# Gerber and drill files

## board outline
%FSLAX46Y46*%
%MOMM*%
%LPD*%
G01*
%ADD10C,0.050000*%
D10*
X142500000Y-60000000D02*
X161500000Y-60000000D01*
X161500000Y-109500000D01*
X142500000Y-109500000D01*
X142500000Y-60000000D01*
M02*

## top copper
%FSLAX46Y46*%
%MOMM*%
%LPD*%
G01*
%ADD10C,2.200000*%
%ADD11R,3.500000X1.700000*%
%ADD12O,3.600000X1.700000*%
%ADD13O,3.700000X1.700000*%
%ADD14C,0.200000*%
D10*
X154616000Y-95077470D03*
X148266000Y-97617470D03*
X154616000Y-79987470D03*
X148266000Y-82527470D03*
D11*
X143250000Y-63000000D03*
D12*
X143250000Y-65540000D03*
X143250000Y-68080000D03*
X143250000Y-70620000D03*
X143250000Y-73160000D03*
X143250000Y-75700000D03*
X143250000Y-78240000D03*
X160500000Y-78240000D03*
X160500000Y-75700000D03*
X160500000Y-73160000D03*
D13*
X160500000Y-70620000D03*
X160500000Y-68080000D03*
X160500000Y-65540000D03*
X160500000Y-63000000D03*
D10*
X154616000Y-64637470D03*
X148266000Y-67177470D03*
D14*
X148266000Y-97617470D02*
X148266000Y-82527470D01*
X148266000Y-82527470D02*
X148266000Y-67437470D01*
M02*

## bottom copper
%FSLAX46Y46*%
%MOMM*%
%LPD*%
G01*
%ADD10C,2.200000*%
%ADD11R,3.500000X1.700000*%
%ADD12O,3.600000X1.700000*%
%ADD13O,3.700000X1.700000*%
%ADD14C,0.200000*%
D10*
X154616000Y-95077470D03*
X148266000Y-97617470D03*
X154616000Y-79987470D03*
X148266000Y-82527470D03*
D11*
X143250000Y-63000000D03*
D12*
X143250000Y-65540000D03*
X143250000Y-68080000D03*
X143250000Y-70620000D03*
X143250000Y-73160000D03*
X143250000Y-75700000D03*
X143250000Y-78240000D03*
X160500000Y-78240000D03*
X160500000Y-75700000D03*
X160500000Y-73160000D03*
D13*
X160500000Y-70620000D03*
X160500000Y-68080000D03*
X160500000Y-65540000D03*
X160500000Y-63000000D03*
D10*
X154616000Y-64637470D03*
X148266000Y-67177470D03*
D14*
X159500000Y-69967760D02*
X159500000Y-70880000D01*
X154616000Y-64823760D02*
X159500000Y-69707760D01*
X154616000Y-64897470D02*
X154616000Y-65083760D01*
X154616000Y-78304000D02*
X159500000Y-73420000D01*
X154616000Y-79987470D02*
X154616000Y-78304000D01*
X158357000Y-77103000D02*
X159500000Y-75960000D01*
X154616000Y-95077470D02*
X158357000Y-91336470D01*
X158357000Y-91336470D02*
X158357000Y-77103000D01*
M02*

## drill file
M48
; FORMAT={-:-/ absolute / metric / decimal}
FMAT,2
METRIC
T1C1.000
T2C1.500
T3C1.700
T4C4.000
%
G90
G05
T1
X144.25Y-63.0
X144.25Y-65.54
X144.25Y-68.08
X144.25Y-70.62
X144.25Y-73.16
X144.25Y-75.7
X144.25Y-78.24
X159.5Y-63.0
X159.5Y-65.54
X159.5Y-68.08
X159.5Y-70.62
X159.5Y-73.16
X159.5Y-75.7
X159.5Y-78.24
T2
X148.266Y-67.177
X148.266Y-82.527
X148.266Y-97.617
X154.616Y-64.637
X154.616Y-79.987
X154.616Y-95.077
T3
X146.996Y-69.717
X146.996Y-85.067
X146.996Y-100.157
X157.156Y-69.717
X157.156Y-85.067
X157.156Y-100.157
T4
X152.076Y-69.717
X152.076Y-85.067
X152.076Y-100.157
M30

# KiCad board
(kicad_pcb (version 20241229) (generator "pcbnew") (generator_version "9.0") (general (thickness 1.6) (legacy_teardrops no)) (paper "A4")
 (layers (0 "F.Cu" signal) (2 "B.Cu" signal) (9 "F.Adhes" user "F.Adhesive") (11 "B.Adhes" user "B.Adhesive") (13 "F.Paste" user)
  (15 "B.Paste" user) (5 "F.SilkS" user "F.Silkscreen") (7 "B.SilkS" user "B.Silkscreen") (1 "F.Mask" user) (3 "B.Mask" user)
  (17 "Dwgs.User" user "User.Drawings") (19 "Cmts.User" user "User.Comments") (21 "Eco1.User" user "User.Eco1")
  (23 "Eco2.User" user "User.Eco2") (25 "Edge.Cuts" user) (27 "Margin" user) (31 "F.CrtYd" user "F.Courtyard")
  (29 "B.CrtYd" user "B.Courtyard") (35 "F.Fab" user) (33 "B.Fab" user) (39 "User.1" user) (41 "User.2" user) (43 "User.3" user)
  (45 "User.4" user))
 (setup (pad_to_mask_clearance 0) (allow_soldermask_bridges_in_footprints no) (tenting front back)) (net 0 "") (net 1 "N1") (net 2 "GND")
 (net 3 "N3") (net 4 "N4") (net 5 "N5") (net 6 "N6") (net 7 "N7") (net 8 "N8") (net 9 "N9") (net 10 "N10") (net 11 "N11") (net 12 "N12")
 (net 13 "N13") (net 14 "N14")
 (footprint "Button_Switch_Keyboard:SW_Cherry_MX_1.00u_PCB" (layer "F.Cu") (at 154.616 95.07747)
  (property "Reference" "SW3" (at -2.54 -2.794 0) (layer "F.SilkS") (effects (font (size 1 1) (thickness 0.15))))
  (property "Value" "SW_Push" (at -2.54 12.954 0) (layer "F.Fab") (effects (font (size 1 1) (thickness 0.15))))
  (pad "" np_thru_hole circle (at -7.62 5.08) (size 1.7 1.7) (drill 1.7) (layers "*.Cu" "*.Mask"))
  (pad "" np_thru_hole circle (at -2.54 5.08) (size 4 4) (drill 4) (layers "*.Cu" "*.Mask"))
  (pad "" np_thru_hole circle (at 2.54 5.08) (size 1.7 1.7) (drill 1.7) (layers "*.Cu" "*.Mask"))
  (pad "1" thru_hole circle (at 0 0) (size 2.2 2.2) (drill 1.5) (layers "*.Cu" "*.Mask") (remove_unused_layers no) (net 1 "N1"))
  (pad "2" thru_hole circle (at -6.35 2.54) (size 2.2 2.2) (drill 1.5) (layers "*.Cu" "*.Mask") (remove_unused_layers no) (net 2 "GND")))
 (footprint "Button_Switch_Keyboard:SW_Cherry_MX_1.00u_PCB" (layer "F.Cu") (at 154.616 79.98747)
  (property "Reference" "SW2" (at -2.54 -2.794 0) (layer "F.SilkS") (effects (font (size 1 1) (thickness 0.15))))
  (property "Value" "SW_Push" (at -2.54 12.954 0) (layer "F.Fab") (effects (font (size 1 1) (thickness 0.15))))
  (pad "" np_thru_hole circle (at -7.62 5.08) (size 1.7 1.7) (drill 1.7) (layers "*.Cu" "*.Mask"))
  (pad "" np_thru_hole circle (at -2.54 5.08) (size 4 4) (drill 4) (layers "*.Cu" "*.Mask"))
  (pad "" np_thru_hole circle (at 2.54 5.08) (size 1.7 1.7) (drill 1.7) (layers "*.Cu" "*.Mask"))
  (pad "1" thru_hole circle (at 0 0) (size 2.2 2.2) (drill 1.5) (layers "*.Cu" "*.Mask") (remove_unused_layers no) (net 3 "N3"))
  (pad "2" thru_hole circle (at -6.35 2.54) (size 2.2 2.2) (drill 1.5) (layers "*.Cu" "*.Mask") (remove_unused_layers no) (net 2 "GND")))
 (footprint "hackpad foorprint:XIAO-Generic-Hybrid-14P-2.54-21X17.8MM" (layer "F.Cu") (at 151.875 70.62)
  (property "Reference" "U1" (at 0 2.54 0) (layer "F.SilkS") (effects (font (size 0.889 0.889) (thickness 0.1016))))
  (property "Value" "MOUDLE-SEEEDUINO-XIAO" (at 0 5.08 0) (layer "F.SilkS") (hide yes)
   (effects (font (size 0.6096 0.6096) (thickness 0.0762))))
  (pad "1" thru_hole rect (at -7.625 -7.62) (size 3.5 1.7) (drill 1 (offset -1 0)) (layers "*.Cu" "*.Mask") (remove_unused_layers no)
   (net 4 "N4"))
  (pad "2" thru_hole oval (at -7.625 -5.08) (size 3.6 1.7) (drill 1 (offset -1 0)) (layers "*.Cu" "*.Mask") (remove_unused_layers no)
   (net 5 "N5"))
  (pad "3" thru_hole oval (at -7.625 -2.54) (size 3.6 1.7) (drill 1 (offset -1 0)) (layers "*.Cu" "*.Mask") (remove_unused_layers no)
   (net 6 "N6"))
  (pad "4" thru_hole oval (at -7.625 0) (size 3.6 1.7) (drill 1 (offset -1 0)) (layers "*.Cu" "*.Mask") (remove_unused_layers no)
   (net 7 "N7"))
  (pad "5" thru_hole oval (at -7.625 2.54) (size 3.6 1.7) (drill 1 (offset -1 0)) (layers "*.Cu" "*.Mask") (remove_unused_layers no)
   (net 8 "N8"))
  (pad "6" thru_hole oval (at -7.625 5.08 180) (size 3.6 1.7) (drill 1 (offset 1 0)) (layers "*.Cu" "*.Mask") (remove_unused_layers no)
   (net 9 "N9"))
  (pad "7" thru_hole oval (at -7.625 7.62) (size 3.6 1.7) (drill 1 (offset -1 0)) (layers "*.Cu" "*.Mask") (remove_unused_layers no)
   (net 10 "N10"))
  (pad "8" thru_hole oval (at 7.625 7.62) (size 3.6 1.7) (drill 1 (offset 1 0)) (layers "*.Cu" "*.Mask") (remove_unused_layers no)
   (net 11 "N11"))
  (pad "9" thru_hole oval (at 7.625 5.08) (size 3.6 1.7) (drill 1 (offset 1 0)) (layers "*.Cu" "*.Mask") (remove_unused_layers no)
   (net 1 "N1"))
  (pad "10" thru_hole oval (at 7.625 2.54) (size 3.6 1.7) (drill 1 (offset 1 0)) (layers "*.Cu" "*.Mask") (remove_unused_layers no)
   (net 3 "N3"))
  (pad "11" thru_hole oval (at 7.625 0) (size 3.7 1.7) (drill 1 (offset 1 0)) (layers "*.Cu" "*.Mask") (remove_unused_layers no)
   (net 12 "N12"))
  (pad "12" thru_hole oval (at 7.625 -2.54) (size 3.7 1.7) (drill 1 (offset 1 0)) (layers "*.Cu" "*.Mask") (remove_unused_layers no)
   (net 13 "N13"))
  (pad "13" thru_hole oval (at 7.625 -5.08) (size 3.7 1.7) (drill 1 (offset 1 0)) (layers "*.Cu" "*.Mask") (remove_unused_layers no)
   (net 2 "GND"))
  (pad "14" thru_hole oval (at 7.625 -7.62) (size 3.7 1.7) (drill 1 (offset 1 0)) (layers "*.Cu" "*.Mask") (remove_unused_layers no)
   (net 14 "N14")))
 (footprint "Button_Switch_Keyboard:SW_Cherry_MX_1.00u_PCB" (layer "F.Cu") (at 154.616 64.63747)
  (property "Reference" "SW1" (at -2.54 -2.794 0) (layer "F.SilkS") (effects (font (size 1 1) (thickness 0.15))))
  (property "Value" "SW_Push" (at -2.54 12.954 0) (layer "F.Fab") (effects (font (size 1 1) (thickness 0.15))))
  (pad "" np_thru_hole circle (at -7.62 5.08) (size 1.7 1.7) (drill 1.7) (layers "*.Cu" "*.Mask"))
  (pad "" np_thru_hole circle (at -2.54 5.08) (size 4 4) (drill 4) (layers "*.Cu" "*.Mask"))
  (pad "" np_thru_hole circle (at 2.54 5.08) (size 1.7 1.7) (drill 1.7) (layers "*.Cu" "*.Mask"))
  (pad "1" thru_hole circle (at 0 0) (size 2.2 2.2) (drill 1.5) (layers "*.Cu" "*.Mask") (remove_unused_layers no) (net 12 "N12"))
  (pad "2" thru_hole circle (at -6.35 2.54) (size 2.2 2.2) (drill 1.5) (layers "*.Cu" "*.Mask") (remove_unused_layers no) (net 2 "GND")))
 (gr_rect (start 142.5 60) (end 161.5 109.5) (stroke (width 0.05) (type default)) (fill no) (layer "Edge.Cuts"))
 (segment (start 159.5 69.96776) (end 159.5 70.88) (width 0.2) (layer "B.Cu") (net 12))
 (segment (start 154.616 64.82376) (end 159.5 69.70776) (width 0.2) (layer "B.Cu") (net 12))
 (segment (start 154.616 64.89747) (end 154.616 65.08376) (width 0.2) (layer "B.Cu") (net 12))
 (segment (start 148.266 97.61747) (end 148.266 82.52747) (width 0.2) (layer "F.Cu") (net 2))
 (segment (start 148.266 82.52747) (end 148.266 67.43747) (width 0.2) (layer "F.Cu") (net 2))
 (segment (start 154.616 78.304) (end 159.5 73.42) (width 0.2) (layer "B.Cu") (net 3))
 (segment (start 154.616 79.98747) (end 154.616 78.304) (width 0.2) (layer "B.Cu") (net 3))
 (segment (start 158.357 77.103) (end 159.5 75.96) (width 0.2) (layer "B.Cu") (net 1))
 (segment (start 154.616 95.07747) (end 158.357 91.33647) (width 0.2) (layer "B.Cu") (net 1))
 (segment (start 158.357 91.33647) (end 158.357 77.103) (width 0.2) (layer "B.Cu") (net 1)))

